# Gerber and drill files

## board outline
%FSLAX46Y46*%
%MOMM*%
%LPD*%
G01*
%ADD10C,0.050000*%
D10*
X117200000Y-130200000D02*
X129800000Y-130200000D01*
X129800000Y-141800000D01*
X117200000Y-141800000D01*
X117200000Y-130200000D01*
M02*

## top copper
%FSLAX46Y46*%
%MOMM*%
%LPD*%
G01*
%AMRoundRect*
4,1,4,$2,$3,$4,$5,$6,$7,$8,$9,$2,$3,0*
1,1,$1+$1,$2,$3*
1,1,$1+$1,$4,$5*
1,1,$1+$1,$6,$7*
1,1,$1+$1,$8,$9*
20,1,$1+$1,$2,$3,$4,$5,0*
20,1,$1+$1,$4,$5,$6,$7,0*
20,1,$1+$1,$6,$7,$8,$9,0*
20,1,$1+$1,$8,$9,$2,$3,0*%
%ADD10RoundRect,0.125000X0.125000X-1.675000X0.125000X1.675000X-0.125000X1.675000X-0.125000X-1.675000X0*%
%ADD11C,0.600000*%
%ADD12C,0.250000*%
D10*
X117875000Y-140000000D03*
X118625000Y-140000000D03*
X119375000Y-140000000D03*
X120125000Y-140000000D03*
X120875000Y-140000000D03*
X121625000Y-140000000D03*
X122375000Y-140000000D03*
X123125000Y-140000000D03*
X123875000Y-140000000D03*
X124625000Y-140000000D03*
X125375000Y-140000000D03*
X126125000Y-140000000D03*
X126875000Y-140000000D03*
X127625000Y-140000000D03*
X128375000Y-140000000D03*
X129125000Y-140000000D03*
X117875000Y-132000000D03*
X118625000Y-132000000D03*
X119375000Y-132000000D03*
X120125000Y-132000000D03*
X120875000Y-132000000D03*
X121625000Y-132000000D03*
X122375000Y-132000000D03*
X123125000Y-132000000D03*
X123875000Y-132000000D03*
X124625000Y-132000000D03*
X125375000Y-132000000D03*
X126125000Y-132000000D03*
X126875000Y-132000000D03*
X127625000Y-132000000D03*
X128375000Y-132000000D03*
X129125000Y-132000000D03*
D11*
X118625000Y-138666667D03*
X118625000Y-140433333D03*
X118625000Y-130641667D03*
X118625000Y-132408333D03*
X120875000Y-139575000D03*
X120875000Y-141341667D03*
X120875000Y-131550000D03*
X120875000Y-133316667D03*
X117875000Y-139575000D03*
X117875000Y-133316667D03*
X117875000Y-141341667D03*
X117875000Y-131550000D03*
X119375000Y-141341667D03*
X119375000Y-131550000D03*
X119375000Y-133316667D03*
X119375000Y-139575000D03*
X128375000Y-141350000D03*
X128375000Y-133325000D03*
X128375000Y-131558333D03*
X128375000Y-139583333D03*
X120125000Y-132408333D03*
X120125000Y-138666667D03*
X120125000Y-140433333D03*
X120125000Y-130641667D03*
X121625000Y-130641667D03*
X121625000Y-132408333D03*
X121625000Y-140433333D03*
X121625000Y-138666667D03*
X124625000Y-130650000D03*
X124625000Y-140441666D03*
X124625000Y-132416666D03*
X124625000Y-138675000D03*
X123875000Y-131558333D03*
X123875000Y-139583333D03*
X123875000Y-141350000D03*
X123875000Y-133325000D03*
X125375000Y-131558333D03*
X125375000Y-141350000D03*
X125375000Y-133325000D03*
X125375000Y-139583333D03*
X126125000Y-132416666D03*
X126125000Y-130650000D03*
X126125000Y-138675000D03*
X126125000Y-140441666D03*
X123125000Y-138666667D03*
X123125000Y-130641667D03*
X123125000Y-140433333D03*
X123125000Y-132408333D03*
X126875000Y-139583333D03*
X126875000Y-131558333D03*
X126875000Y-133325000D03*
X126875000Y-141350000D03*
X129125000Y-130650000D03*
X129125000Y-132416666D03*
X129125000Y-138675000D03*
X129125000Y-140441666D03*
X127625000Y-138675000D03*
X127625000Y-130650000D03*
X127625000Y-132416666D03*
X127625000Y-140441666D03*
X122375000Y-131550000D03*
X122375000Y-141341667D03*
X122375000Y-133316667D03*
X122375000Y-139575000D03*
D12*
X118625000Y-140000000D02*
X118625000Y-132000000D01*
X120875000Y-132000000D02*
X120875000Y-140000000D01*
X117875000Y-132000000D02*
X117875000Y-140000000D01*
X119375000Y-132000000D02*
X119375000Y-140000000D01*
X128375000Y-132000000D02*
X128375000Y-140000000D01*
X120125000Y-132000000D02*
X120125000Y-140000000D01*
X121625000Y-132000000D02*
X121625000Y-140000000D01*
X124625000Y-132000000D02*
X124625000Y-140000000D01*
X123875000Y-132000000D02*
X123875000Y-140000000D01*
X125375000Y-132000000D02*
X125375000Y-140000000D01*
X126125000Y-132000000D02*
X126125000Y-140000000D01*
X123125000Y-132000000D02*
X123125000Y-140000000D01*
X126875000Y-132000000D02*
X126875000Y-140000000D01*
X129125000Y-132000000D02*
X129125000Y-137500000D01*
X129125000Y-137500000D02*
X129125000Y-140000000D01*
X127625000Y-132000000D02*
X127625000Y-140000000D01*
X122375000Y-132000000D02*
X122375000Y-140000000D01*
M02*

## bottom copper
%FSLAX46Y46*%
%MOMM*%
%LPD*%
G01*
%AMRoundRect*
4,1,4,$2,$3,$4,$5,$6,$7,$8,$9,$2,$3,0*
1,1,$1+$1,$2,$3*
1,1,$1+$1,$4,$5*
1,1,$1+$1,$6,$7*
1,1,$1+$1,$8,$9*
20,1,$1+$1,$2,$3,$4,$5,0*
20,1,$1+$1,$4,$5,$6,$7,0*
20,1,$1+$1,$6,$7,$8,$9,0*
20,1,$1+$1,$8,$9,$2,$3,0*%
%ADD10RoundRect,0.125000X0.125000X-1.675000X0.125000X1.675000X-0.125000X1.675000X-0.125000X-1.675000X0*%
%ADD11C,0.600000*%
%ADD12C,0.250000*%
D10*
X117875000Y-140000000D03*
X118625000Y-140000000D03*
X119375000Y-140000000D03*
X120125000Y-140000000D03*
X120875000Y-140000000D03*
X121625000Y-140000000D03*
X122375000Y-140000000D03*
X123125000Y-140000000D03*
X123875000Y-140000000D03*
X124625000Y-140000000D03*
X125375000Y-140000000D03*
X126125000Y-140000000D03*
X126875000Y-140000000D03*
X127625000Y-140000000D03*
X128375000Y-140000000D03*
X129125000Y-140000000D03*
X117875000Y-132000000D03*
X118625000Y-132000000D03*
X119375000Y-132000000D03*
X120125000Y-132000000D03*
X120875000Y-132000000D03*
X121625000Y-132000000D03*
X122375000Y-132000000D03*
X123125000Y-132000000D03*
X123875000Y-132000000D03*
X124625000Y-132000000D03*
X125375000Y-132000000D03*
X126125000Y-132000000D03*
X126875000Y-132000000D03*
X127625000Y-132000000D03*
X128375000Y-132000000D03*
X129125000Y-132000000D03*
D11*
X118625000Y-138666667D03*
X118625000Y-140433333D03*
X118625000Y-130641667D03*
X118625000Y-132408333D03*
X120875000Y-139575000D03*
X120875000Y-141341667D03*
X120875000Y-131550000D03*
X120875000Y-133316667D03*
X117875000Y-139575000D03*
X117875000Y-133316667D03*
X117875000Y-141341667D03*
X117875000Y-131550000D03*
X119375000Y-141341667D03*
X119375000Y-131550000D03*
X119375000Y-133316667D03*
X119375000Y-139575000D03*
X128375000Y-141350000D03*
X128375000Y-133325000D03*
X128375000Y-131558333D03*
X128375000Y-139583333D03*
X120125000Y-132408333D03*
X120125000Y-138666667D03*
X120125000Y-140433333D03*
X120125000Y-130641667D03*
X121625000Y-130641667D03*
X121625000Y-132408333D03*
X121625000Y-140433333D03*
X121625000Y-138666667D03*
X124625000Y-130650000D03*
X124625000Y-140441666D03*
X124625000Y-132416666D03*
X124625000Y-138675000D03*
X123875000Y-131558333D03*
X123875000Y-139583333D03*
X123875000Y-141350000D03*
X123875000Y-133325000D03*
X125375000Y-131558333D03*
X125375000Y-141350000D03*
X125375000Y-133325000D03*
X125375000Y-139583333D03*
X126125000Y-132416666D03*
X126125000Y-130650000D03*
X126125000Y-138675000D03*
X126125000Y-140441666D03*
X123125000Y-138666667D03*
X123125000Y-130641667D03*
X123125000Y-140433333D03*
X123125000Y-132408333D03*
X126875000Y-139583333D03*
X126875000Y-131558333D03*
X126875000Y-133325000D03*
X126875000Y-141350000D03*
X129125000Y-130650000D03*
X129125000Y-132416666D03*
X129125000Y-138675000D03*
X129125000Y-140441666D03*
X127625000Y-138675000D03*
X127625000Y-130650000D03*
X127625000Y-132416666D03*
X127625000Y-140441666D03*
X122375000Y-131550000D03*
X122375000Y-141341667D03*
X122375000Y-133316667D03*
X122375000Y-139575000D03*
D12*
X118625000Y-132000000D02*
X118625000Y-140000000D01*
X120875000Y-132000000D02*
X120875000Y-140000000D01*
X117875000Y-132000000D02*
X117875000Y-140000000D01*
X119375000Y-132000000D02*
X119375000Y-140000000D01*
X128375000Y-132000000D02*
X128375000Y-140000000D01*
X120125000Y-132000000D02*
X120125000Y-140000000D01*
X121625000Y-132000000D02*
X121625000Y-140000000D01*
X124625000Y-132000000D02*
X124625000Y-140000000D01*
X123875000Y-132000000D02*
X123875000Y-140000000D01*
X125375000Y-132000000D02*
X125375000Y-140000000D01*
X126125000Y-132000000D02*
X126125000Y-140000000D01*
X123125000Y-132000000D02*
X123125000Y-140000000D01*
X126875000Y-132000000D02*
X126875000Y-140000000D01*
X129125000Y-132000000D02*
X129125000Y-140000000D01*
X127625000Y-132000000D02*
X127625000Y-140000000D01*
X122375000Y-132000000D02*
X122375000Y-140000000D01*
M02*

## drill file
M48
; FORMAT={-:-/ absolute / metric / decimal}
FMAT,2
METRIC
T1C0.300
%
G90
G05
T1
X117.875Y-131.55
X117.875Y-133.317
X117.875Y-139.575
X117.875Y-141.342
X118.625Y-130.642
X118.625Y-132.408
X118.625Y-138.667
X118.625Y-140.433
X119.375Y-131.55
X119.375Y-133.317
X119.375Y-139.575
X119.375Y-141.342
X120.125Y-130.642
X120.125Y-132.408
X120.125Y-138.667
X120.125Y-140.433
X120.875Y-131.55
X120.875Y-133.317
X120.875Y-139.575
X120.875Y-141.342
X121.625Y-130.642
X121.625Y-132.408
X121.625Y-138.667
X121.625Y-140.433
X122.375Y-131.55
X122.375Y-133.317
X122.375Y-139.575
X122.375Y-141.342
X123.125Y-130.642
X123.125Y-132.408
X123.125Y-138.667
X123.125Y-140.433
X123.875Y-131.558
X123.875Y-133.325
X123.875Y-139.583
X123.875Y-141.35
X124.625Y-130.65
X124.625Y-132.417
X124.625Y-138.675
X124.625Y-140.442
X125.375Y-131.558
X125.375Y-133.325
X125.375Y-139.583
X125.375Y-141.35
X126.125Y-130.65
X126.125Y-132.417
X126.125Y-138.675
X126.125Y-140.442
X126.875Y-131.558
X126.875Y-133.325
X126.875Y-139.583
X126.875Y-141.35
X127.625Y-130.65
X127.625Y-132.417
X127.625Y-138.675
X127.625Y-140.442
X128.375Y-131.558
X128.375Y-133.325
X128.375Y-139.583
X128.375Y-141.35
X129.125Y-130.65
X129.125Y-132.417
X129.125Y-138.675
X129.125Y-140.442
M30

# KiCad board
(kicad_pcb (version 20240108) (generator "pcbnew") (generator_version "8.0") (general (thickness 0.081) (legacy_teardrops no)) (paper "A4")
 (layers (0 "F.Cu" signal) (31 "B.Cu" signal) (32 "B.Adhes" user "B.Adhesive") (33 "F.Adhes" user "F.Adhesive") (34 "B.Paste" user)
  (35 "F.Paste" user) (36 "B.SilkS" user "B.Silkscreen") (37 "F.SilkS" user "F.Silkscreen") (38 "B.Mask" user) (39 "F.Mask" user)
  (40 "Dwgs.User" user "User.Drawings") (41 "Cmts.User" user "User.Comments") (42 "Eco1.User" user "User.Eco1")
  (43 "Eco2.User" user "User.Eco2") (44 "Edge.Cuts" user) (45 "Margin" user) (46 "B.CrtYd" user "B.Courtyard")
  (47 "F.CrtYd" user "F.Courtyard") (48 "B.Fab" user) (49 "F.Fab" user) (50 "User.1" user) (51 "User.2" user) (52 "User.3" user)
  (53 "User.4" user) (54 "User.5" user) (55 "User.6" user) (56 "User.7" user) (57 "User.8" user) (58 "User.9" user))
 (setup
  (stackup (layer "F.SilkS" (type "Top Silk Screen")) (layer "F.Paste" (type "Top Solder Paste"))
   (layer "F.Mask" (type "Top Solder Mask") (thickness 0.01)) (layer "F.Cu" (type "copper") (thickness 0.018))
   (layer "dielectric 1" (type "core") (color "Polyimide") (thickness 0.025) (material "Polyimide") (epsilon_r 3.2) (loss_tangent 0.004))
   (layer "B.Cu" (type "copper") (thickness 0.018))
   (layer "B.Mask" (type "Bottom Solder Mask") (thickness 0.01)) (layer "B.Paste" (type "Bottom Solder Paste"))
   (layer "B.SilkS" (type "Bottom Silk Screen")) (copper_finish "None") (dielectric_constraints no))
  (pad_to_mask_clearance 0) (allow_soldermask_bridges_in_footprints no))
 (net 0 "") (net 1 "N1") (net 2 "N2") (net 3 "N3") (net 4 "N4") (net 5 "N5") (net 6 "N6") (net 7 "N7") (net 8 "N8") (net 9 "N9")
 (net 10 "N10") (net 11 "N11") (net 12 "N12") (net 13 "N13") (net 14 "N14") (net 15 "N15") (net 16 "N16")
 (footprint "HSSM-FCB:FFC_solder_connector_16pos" (layer "F.Cu") (at 123.5 140)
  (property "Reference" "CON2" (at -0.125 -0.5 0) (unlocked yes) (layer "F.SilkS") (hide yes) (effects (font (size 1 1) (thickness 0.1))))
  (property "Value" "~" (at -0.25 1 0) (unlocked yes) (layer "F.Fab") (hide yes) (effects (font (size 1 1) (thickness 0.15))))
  (pad "1" smd roundrect (at -5.625 0 90) (size 3.6 0.5) (layers "F.Cu" "F.Mask") (roundrect_rratio 0.25) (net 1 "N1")
   (thermal_bridge_angle 45))
  (pad "1" smd roundrect (at -5.625 0 90) (size 3.6 0.5) (layers "B.Cu" "B.Mask") (roundrect_rratio 0.25) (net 1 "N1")
   (thermal_bridge_angle 45))
  (pad "2" smd roundrect (at -4.875 0 90) (size 3.6 0.5) (layers "F.Cu" "F.Mask") (roundrect_rratio 0.25) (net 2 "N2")
   (thermal_bridge_angle 45))
  (pad "2" smd roundrect (at -4.875 0 90) (size 3.6 0.5) (layers "B.Cu" "B.Mask") (roundrect_rratio 0.25) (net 2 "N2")
   (thermal_bridge_angle 45))
  (pad "3" smd roundrect (at -4.125 0 90) (size 3.6 0.5) (layers "F.Cu" "F.Mask") (roundrect_rratio 0.25) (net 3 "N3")
   (thermal_bridge_angle 45))
  (pad "3" smd roundrect (at -4.125 0 90) (size 3.6 0.5) (layers "B.Cu" "B.Mask") (roundrect_rratio 0.25) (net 3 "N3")
   (thermal_bridge_angle 45))
  (pad "4" smd roundrect (at -3.375 0 90) (size 3.6 0.5) (layers "F.Cu" "F.Mask") (roundrect_rratio 0.25) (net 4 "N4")
   (thermal_bridge_angle 45))
  (pad "4" smd roundrect (at -3.375 0 90) (size 3.6 0.5) (layers "B.Cu" "B.Mask") (roundrect_rratio 0.25) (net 4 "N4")
   (thermal_bridge_angle 45))
  (pad "5" smd roundrect (at -2.625 0 90) (size 3.6 0.5) (layers "F.Cu" "F.Mask") (roundrect_rratio 0.25) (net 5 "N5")
   (thermal_bridge_angle 45))
  (pad "5" smd roundrect (at -2.625 0 90) (size 3.6 0.5) (layers "B.Cu" "B.Mask") (roundrect_rratio 0.25) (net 5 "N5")
   (thermal_bridge_angle 45))
  (pad "6" smd roundrect (at -1.875 0 90) (size 3.6 0.5) (layers "F.Cu" "F.Mask") (roundrect_rratio 0.25) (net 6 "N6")
   (thermal_bridge_angle 45))
  (pad "6" smd roundrect (at -1.875 0 90) (size 3.6 0.5) (layers "B.Cu" "B.Mask") (roundrect_rratio 0.25) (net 6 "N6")
   (thermal_bridge_angle 45))
  (pad "7" smd roundrect (at -1.125 0 90) (size 3.6 0.5) (layers "F.Cu" "F.Mask") (roundrect_rratio 0.25) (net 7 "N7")
   (thermal_bridge_angle 45))
  (pad "7" smd roundrect (at -1.125 0 90) (size 3.6 0.5) (layers "B.Cu" "B.Mask") (roundrect_rratio 0.25) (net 7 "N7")
   (thermal_bridge_angle 45))
  (pad "8" smd roundrect (at -0.375 0 90) (size 3.6 0.5) (layers "F.Cu" "F.Mask") (roundrect_rratio 0.25) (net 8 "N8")
   (thermal_bridge_angle 45))
  (pad "8" smd roundrect (at -0.375 0 90) (size 3.6 0.5) (layers "B.Cu" "B.Mask") (roundrect_rratio 0.25) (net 8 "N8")
   (thermal_bridge_angle 45))
  (pad "9" smd roundrect (at 0.375 0 90) (size 3.6 0.5) (layers "F.Cu" "F.Mask") (roundrect_rratio 0.25) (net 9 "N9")
   (thermal_bridge_angle 45))
  (pad "9" smd roundrect (at 0.375 0 90) (size 3.6 0.5) (layers "B.Cu" "B.Mask") (roundrect_rratio 0.25) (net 9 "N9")
   (thermal_bridge_angle 45))
  (pad "10" smd roundrect (at 1.125 0 90) (size 3.6 0.5) (layers "F.Cu" "F.Mask") (roundrect_rratio 0.25) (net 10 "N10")
   (thermal_bridge_angle 45))
  (pad "10" smd roundrect (at 1.125 0 90) (size 3.6 0.5) (layers "B.Cu" "B.Mask") (roundrect_rratio 0.25) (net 10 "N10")
   (thermal_bridge_angle 45))
  (pad "11" smd roundrect (at 1.875 0 90) (size 3.6 0.5) (layers "F.Cu" "F.Mask") (roundrect_rratio 0.25) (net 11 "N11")
   (thermal_bridge_angle 45))
  (pad "11" smd roundrect (at 1.875 0 90) (size 3.6 0.5) (layers "B.Cu" "B.Mask") (roundrect_rratio 0.25) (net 11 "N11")
   (thermal_bridge_angle 45))
  (pad "12" smd roundrect (at 2.625 0 90) (size 3.6 0.5) (layers "F.Cu" "F.Mask") (roundrect_rratio 0.25) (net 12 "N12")
   (thermal_bridge_angle 45))
  (pad "12" smd roundrect (at 2.625 0 90) (size 3.6 0.5) (layers "B.Cu" "B.Mask") (roundrect_rratio 0.25) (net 12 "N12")
   (thermal_bridge_angle 45))
  (pad "13" smd roundrect (at 3.375 0 90) (size 3.6 0.5) (layers "F.Cu" "F.Mask") (roundrect_rratio 0.25) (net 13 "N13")
   (thermal_bridge_angle 45))
  (pad "13" smd roundrect (at 3.375 0 90) (size 3.6 0.5) (layers "B.Cu" "B.Mask") (roundrect_rratio 0.25) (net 13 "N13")
   (thermal_bridge_angle 45))
  (pad "14" smd roundrect (at 4.125 0 90) (size 3.6 0.5) (layers "F.Cu" "F.Mask") (roundrect_rratio 0.25) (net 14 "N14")
   (thermal_bridge_angle 45))
  (pad "14" smd roundrect (at 4.125 0 90) (size 3.6 0.5) (layers "B.Cu" "B.Mask") (roundrect_rratio 0.25) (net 14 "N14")
   (thermal_bridge_angle 45))
  (pad "15" smd roundrect (at 4.875 0 90) (size 3.6 0.5) (layers "F.Cu" "F.Mask") (roundrect_rratio 0.25) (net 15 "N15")
   (thermal_bridge_angle 45))
  (pad "15" smd roundrect (at 4.875 0 90) (size 3.6 0.5) (layers "B.Cu" "B.Mask") (roundrect_rratio 0.25) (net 15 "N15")
   (thermal_bridge_angle 45))
  (pad "16" smd roundrect (at 5.625 0 90) (size 3.6 0.5) (layers "F.Cu" "F.Mask") (roundrect_rratio 0.25) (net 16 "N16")
   (thermal_bridge_angle 45))
  (pad "16" smd roundrect (at 5.625 0 90) (size 3.6 0.5) (layers "B.Cu" "B.Mask") (roundrect_rratio 0.25) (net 16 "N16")
   (thermal_bridge_angle 45)))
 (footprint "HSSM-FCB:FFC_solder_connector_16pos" (layer "F.Cu") (at 123.5 132)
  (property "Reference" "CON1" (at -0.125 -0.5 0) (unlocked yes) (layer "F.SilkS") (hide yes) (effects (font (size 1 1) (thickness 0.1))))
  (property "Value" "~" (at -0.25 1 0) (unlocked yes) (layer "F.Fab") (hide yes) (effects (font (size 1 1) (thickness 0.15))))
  (pad "1" smd roundrect (at -5.625 0 90) (size 3.6 0.5) (layers "F.Cu" "F.Mask") (roundrect_rratio 0.25) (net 1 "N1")
   (thermal_bridge_angle 45))
  (pad "1" smd roundrect (at -5.625 0 90) (size 3.6 0.5) (layers "B.Cu" "B.Mask") (roundrect_rratio 0.25) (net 1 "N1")
   (thermal_bridge_angle 45))
  (pad "2" smd roundrect (at -4.875 0 90) (size 3.6 0.5) (layers "F.Cu" "F.Mask") (roundrect_rratio 0.25) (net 2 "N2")
   (thermal_bridge_angle 45))
  (pad "2" smd roundrect (at -4.875 0 90) (size 3.6 0.5) (layers "B.Cu" "B.Mask") (roundrect_rratio 0.25) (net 2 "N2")
   (thermal_bridge_angle 45))
  (pad "3" smd roundrect (at -4.125 0 90) (size 3.6 0.5) (layers "F.Cu" "F.Mask") (roundrect_rratio 0.25) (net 3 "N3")
   (thermal_bridge_angle 45))
  (pad "3" smd roundrect (at -4.125 0 90) (size 3.6 0.5) (layers "B.Cu" "B.Mask") (roundrect_rratio 0.25) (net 3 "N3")
   (thermal_bridge_angle 45))
  (pad "4" smd roundrect (at -3.375 0 90) (size 3.6 0.5) (layers "F.Cu" "F.Mask") (roundrect_rratio 0.25) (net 4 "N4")
   (thermal_bridge_angle 45))
  (pad "4" smd roundrect (at -3.375 0 90) (size 3.6 0.5) (layers "B.Cu" "B.Mask") (roundrect_rratio 0.25) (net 4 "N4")
   (thermal_bridge_angle 45))
  (pad "5" smd roundrect (at -2.625 0 90) (size 3.6 0.5) (layers "F.Cu" "F.Mask") (roundrect_rratio 0.25) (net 5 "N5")
   (thermal_bridge_angle 45))
  (pad "5" smd roundrect (at -2.625 0 90) (size 3.6 0.5) (layers "B.Cu" "B.Mask") (roundrect_rratio 0.25) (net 5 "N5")
   (thermal_bridge_angle 45))
  (pad "6" smd roundrect (at -1.875 0 90) (size 3.6 0.5) (layers "F.Cu" "F.Mask") (roundrect_rratio 0.25) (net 6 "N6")
   (thermal_bridge_angle 45))
  (pad "6" smd roundrect (at -1.875 0 90) (size 3.6 0.5) (layers "B.Cu" "B.Mask") (roundrect_rratio 0.25) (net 6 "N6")
   (thermal_bridge_angle 45))
  (pad "7" smd roundrect (at -1.125 0 90) (size 3.6 0.5) (layers "F.Cu" "F.Mask") (roundrect_rratio 0.25) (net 7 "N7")
   (thermal_bridge_angle 45))
  (pad "7" smd roundrect (at -1.125 0 90) (size 3.6 0.5) (layers "B.Cu" "B.Mask") (roundrect_rratio 0.25) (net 7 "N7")
   (thermal_bridge_angle 45))
  (pad "8" smd roundrect (at -0.375 0 90) (size 3.6 0.5) (layers "F.Cu" "F.Mask") (roundrect_rratio 0.25) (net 8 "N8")
   (thermal_bridge_angle 45))
  (pad "8" smd roundrect (at -0.375 0 90) (size 3.6 0.5) (layers "B.Cu" "B.Mask") (roundrect_rratio 0.25) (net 8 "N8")
   (thermal_bridge_angle 45))
  (pad "9" smd roundrect (at 0.375 0 90) (size 3.6 0.5) (layers "F.Cu" "F.Mask") (roundrect_rratio 0.25) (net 9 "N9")
   (thermal_bridge_angle 45))
  (pad "9" smd roundrect (at 0.375 0 90) (size 3.6 0.5) (layers "B.Cu" "B.Mask") (roundrect_rratio 0.25) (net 9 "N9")
   (thermal_bridge_angle 45))
  (pad "10" smd roundrect (at 1.125 0 90) (size 3.6 0.5) (layers "F.Cu" "F.Mask") (roundrect_rratio 0.25) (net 10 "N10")
   (thermal_bridge_angle 45))
  (pad "10" smd roundrect (at 1.125 0 90) (size 3.6 0.5) (layers "B.Cu" "B.Mask") (roundrect_rratio 0.25) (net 10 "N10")
   (thermal_bridge_angle 45))
  (pad "11" smd roundrect (at 1.875 0 90) (size 3.6 0.5) (layers "F.Cu" "F.Mask") (roundrect_rratio 0.25) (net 11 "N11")
   (thermal_bridge_angle 45))
  (pad "11" smd roundrect (at 1.875 0 90) (size 3.6 0.5) (layers "B.Cu" "B.Mask") (roundrect_rratio 0.25) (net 11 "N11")
   (thermal_bridge_angle 45))
  (pad "12" smd roundrect (at 2.625 0 90) (size 3.6 0.5) (layers "F.Cu" "F.Mask") (roundrect_rratio 0.25) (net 12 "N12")
   (thermal_bridge_angle 45))
  (pad "12" smd roundrect (at 2.625 0 90) (size 3.6 0.5) (layers "B.Cu" "B.Mask") (roundrect_rratio 0.25) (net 12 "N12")
   (thermal_bridge_angle 45))
  (pad "13" smd roundrect (at 3.375 0 90) (size 3.6 0.5) (layers "F.Cu" "F.Mask") (roundrect_rratio 0.25) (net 13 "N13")
   (thermal_bridge_angle 45))
  (pad "13" smd roundrect (at 3.375 0 90) (size 3.6 0.5) (layers "B.Cu" "B.Mask") (roundrect_rratio 0.25) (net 13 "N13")
   (thermal_bridge_angle 45))
  (pad "14" smd roundrect (at 4.125 0 90) (size 3.6 0.5) (layers "F.Cu" "F.Mask") (roundrect_rratio 0.25) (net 14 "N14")
   (thermal_bridge_angle 45))
  (pad "14" smd roundrect (at 4.125 0 90) (size 3.6 0.5) (layers "B.Cu" "B.Mask") (roundrect_rratio 0.25) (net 14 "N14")
   (thermal_bridge_angle 45))
  (pad "15" smd roundrect (at 4.875 0 90) (size 3.6 0.5) (layers "F.Cu" "F.Mask") (roundrect_rratio 0.25) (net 15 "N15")
   (thermal_bridge_angle 45))
  (pad "15" smd roundrect (at 4.875 0 90) (size 3.6 0.5) (layers "B.Cu" "B.Mask") (roundrect_rratio 0.25) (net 15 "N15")
   (thermal_bridge_angle 45))
  (pad "16" smd roundrect (at 5.625 0 90) (size 3.6 0.5) (layers "F.Cu" "F.Mask") (roundrect_rratio 0.25) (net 16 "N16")
   (thermal_bridge_angle 45))
  (pad "16" smd roundrect (at 5.625 0 90) (size 3.6 0.5) (layers "B.Cu" "B.Mask") (roundrect_rratio 0.25) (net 16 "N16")
   (thermal_bridge_angle 45)))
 (gr_rect (start 117.2 130.2) (end 129.8 141.8) (stroke (width 0.05) (type default)) (fill none) (layer "Edge.Cuts"))
 (segment (start 118.625 140) (end 118.625 132) (width 0.25) (layer "F.Cu") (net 2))
 (via (at 118.625 138.666667) (size 0.6) (drill 0.3) (layers "F.Cu" "B.Cu") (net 2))
 (via (at 118.625 140.433333) (size 0.6) (drill 0.3) (layers "F.Cu" "B.Cu") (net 2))
 (via (at 118.625 130.641667) (size 0.6) (drill 0.3) (layers "F.Cu" "B.Cu") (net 2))
 (via (at 118.625 132.408333) (size 0.6) (drill 0.3) (layers "F.Cu" "B.Cu") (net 2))
 (segment (start 118.625 132) (end 118.625 140) (width 0.25) (layer "B.Cu") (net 2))
 (segment (start 120.875 132) (end 120.875 140) (width 0.25) (layer "F.Cu") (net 5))
 (via (at 120.875 139.575) (size 0.6) (drill 0.3) (layers "F.Cu" "B.Cu") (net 5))
 (via (at 120.875 141.341667) (size 0.6) (drill 0.3) (layers "F.Cu" "B.Cu") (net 5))
 (via (at 120.875 131.55) (size 0.6) (drill 0.3) (layers "F.Cu" "B.Cu") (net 5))
 (via (at 120.875 133.316667) (size 0.6) (drill 0.3) (layers "F.Cu" "B.Cu") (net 5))
 (segment (start 120.875 132) (end 120.875 140) (width 0.25) (layer "B.Cu") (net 5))
 (segment (start 117.875 132) (end 117.875 140) (width 0.25) (layer "F.Cu") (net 1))
 (via (at 117.875 139.575) (size 0.6) (drill 0.3) (layers "F.Cu" "B.Cu") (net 1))
 (via (at 117.875 133.316667) (size 0.6) (drill 0.3) (layers "F.Cu" "B.Cu") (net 1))
 (via (at 117.875 141.341667) (size 0.6) (drill 0.3) (layers "F.Cu" "B.Cu") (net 1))
 (via (at 117.875 131.55) (size 0.6) (drill 0.3) (layers "F.Cu" "B.Cu") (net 1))
 (segment (start 117.875 132) (end 117.875 140) (width 0.25) (layer "B.Cu") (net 1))
 (segment (start 119.375 132) (end 119.375 140) (width 0.25) (layer "F.Cu") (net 3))
 (via (at 119.375 141.341667) (size 0.6) (drill 0.3) (layers "F.Cu" "B.Cu") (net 3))
 (via (at 119.375 131.55) (size 0.6) (drill 0.3) (layers "F.Cu" "B.Cu") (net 3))
 (via (at 119.375 133.316667) (size 0.6) (drill 0.3) (layers "F.Cu" "B.Cu") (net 3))
 (via (at 119.375 139.575) (size 0.6) (drill 0.3) (layers "F.Cu" "B.Cu") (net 3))
 (segment (start 119.375 132) (end 119.375 140) (width 0.25) (layer "B.Cu") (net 3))
 (segment (start 128.375 132) (end 128.375 140) (width 0.25) (layer "F.Cu") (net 15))
 (via (at 128.375 141.35) (size 0.6) (drill 0.3) (layers "F.Cu" "B.Cu") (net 15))
 (via (at 128.375 133.325) (size 0.6) (drill 0.3) (layers "F.Cu" "B.Cu") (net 15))
 (via (at 128.375 131.558333) (size 0.6) (drill 0.3) (layers "F.Cu" "B.Cu") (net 15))
 (via (at 128.375 139.583333) (size 0.6) (drill 0.3) (layers "F.Cu" "B.Cu") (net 15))
 (segment (start 128.375 132) (end 128.375 140) (width 0.25) (layer "B.Cu") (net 15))
 (segment (start 120.125 132) (end 120.125 140) (width 0.25) (layer "F.Cu") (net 4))
 (via (at 120.125 132.408333) (size 0.6) (drill 0.3) (layers "F.Cu" "B.Cu") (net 4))
 (via (at 120.125 138.666667) (size 0.6) (drill 0.3) (layers "F.Cu" "B.Cu") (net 4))
 (via (at 120.125 140.433333) (size 0.6) (drill 0.3) (layers "F.Cu" "B.Cu") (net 4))
 (via (at 120.125 130.641667) (size 0.6) (drill 0.3) (layers "F.Cu" "B.Cu") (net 4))
 (segment (start 120.125 132) (end 120.125 140) (width 0.25) (layer "B.Cu") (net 4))
 (segment (start 121.625 132) (end 121.625 140) (width 0.25) (layer "F.Cu") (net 6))
 (via (at 121.625 130.641667) (size 0.6) (drill 0.3) (layers "F.Cu" "B.Cu") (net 6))
 (via (at 121.625 132.408333) (size 0.6) (drill 0.3) (layers "F.Cu" "B.Cu") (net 6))
 (via (at 121.625 140.433333) (size 0.6) (drill 0.3) (layers "F.Cu" "B.Cu") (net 6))
 (via (at 121.625 138.666667) (size 0.6) (drill 0.3) (layers "F.Cu" "B.Cu") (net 6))
 (segment (start 121.625 132) (end 121.625 140) (width 0.25) (layer "B.Cu") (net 6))
 (segment (start 124.625 132) (end 124.625 140) (width 0.25) (layer "F.Cu") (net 10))
 (via (at 124.625 130.65) (size 0.6) (drill 0.3) (layers "F.Cu" "B.Cu") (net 10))
 (via (at 124.625 140.441666) (size 0.6) (drill 0.3) (layers "F.Cu" "B.Cu") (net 10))
 (via (at 124.625 132.416666) (size 0.6) (drill 0.3) (layers "F.Cu" "B.Cu") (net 10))
 (via (at 124.625 138.675) (size 0.6) (drill 0.3) (layers "F.Cu" "B.Cu") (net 10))
 (segment (start 124.625 132) (end 124.625 140) (width 0.25) (layer "B.Cu") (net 10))
 (segment (start 123.875 132) (end 123.875 140) (width 0.25) (layer "F.Cu") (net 9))
 (via (at 123.875 131.558333) (size 0.6) (drill 0.3) (layers "F.Cu" "B.Cu") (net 9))
 (via (at 123.875 139.583333) (size 0.6) (drill 0.3) (layers "F.Cu" "B.Cu") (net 9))
 (via (at 123.875 141.35) (size 0.6) (drill 0.3) (layers "F.Cu" "B.Cu") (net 9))
 (via (at 123.875 133.325) (size 0.6) (drill 0.3) (layers "F.Cu" "B.Cu") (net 9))
 (segment (start 123.875 132) (end 123.875 140) (width 0.25) (layer "B.Cu") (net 9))
 (segment (start 125.375 132) (end 125.375 140) (width 0.25) (layer "F.Cu") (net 11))
 (via (at 125.375 131.558333) (size 0.6) (drill 0.3) (layers "F.Cu" "B.Cu") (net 11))
 (via (at 125.375 141.35) (size 0.6) (drill 0.3) (layers "F.Cu" "B.Cu") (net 11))
 (via (at 125.375 133.325) (size 0.6) (drill 0.3) (layers "F.Cu" "B.Cu") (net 11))
 (via (at 125.375 139.583333) (size 0.6) (drill 0.3) (layers "F.Cu" "B.Cu") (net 11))
 (segment (start 125.375 132) (end 125.375 140) (width 0.25) (layer "B.Cu") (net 11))
 (segment (start 126.125 132) (end 126.125 140) (width 0.25) (layer "F.Cu") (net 12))
 (via (at 126.125 132.416666) (size 0.6) (drill 0.3) (layers "F.Cu" "B.Cu") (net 12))
 (via (at 126.125 130.65) (size 0.6) (drill 0.3) (layers "F.Cu" "B.Cu") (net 12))
 (via (at 126.125 138.675) (size 0.6) (drill 0.3) (layers "F.Cu" "B.Cu") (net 12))
 (via (at 126.125 140.441666) (size 0.6) (drill 0.3) (layers "F.Cu" "B.Cu") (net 12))
 (segment (start 126.125 132) (end 126.125 140) (width 0.25) (layer "B.Cu") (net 12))
 (segment (start 123.125 132) (end 123.125 140) (width 0.25) (layer "F.Cu") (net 8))
 (via (at 123.125 138.666667) (size 0.6) (drill 0.3) (layers "F.Cu" "B.Cu") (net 8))
 (via (at 123.125 130.641667) (size 0.6) (drill 0.3) (layers "F.Cu" "B.Cu") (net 8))
 (via (at 123.125 140.433333) (size 0.6) (drill 0.3) (layers "F.Cu" "B.Cu") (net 8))
 (via (at 123.125 132.408333) (size 0.6) (drill 0.3) (layers "F.Cu" "B.Cu") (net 8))
 (segment (start 123.125 132) (end 123.125 140) (width 0.25) (layer "B.Cu") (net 8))
 (segment (start 126.875 132) (end 126.875 140) (width 0.25) (layer "F.Cu") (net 13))
 (via (at 126.875 139.583333) (size 0.6) (drill 0.3) (layers "F.Cu" "B.Cu") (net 13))
 (via (at 126.875 131.558333) (size 0.6) (drill 0.3) (layers "F.Cu" "B.Cu") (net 13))
 (via (at 126.875 133.325) (size 0.6) (drill 0.3) (layers "F.Cu" "B.Cu") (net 13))
 (via (at 126.875 141.35) (size 0.6) (drill 0.3) (layers "F.Cu" "B.Cu") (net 13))
 (segment (start 126.875 132) (end 126.875 140) (width 0.25) (layer "B.Cu") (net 13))
 (segment (start 129.125 132) (end 129.125 137.5) (width 0.25) (layer "F.Cu") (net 16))
 (segment (start 129.125 137.5) (end 129.125 140) (width 0.25) (layer "F.Cu") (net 16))
 (via (at 129.125 130.65) (size 0.6) (drill 0.3) (layers "F.Cu" "B.Cu") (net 16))
 (via (at 129.125 132.416666) (size 0.6) (drill 0.3) (layers "F.Cu" "B.Cu") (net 16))
 (via (at 129.125 138.675) (size 0.6) (drill 0.3) (layers "F.Cu" "B.Cu") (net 16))
 (via (at 129.125 140.441666) (size 0.6) (drill 0.3) (layers "F.Cu" "B.Cu") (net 16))
 (segment (start 129.125 132) (end 129.125 140) (width 0.25) (layer "B.Cu") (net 16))
 (segment (start 127.625 132) (end 127.625 140) (width 0.25) (layer "F.Cu") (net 14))
 (via (at 127.625 138.675) (size 0.6) (drill 0.3) (layers "F.Cu" "B.Cu") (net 14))
 (via (at 127.625 130.65) (size 0.6) (drill 0.3) (layers "F.Cu" "B.Cu") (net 14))
 (via (at 127.625 132.416666) (size 0.6) (drill 0.3) (layers "F.Cu" "B.Cu") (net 14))
 (via (at 127.625 140.441666) (size 0.6) (drill 0.3) (layers "F.Cu" "B.Cu") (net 14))
 (segment (start 127.625 132) (end 127.625 140) (width 0.25) (layer "B.Cu") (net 14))
 (segment (start 122.375 132) (end 122.375 140) (width 0.25) (layer "F.Cu") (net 7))
 (via (at 122.375 131.55) (size 0.6) (drill 0.3) (layers "F.Cu" "B.Cu") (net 7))
 (via (at 122.375 141.341667) (size 0.6) (drill 0.3) (layers "F.Cu" "B.Cu") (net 7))
 (via (at 122.375 133.316667) (size 0.6) (drill 0.3) (layers "F.Cu" "B.Cu") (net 7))
 (via (at 122.375 139.575) (size 0.6) (drill 0.3) (layers "F.Cu" "B.Cu") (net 7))
 (segment (start 122.375 132) (end 122.375 140) (width 0.25) (layer "B.Cu") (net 7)))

